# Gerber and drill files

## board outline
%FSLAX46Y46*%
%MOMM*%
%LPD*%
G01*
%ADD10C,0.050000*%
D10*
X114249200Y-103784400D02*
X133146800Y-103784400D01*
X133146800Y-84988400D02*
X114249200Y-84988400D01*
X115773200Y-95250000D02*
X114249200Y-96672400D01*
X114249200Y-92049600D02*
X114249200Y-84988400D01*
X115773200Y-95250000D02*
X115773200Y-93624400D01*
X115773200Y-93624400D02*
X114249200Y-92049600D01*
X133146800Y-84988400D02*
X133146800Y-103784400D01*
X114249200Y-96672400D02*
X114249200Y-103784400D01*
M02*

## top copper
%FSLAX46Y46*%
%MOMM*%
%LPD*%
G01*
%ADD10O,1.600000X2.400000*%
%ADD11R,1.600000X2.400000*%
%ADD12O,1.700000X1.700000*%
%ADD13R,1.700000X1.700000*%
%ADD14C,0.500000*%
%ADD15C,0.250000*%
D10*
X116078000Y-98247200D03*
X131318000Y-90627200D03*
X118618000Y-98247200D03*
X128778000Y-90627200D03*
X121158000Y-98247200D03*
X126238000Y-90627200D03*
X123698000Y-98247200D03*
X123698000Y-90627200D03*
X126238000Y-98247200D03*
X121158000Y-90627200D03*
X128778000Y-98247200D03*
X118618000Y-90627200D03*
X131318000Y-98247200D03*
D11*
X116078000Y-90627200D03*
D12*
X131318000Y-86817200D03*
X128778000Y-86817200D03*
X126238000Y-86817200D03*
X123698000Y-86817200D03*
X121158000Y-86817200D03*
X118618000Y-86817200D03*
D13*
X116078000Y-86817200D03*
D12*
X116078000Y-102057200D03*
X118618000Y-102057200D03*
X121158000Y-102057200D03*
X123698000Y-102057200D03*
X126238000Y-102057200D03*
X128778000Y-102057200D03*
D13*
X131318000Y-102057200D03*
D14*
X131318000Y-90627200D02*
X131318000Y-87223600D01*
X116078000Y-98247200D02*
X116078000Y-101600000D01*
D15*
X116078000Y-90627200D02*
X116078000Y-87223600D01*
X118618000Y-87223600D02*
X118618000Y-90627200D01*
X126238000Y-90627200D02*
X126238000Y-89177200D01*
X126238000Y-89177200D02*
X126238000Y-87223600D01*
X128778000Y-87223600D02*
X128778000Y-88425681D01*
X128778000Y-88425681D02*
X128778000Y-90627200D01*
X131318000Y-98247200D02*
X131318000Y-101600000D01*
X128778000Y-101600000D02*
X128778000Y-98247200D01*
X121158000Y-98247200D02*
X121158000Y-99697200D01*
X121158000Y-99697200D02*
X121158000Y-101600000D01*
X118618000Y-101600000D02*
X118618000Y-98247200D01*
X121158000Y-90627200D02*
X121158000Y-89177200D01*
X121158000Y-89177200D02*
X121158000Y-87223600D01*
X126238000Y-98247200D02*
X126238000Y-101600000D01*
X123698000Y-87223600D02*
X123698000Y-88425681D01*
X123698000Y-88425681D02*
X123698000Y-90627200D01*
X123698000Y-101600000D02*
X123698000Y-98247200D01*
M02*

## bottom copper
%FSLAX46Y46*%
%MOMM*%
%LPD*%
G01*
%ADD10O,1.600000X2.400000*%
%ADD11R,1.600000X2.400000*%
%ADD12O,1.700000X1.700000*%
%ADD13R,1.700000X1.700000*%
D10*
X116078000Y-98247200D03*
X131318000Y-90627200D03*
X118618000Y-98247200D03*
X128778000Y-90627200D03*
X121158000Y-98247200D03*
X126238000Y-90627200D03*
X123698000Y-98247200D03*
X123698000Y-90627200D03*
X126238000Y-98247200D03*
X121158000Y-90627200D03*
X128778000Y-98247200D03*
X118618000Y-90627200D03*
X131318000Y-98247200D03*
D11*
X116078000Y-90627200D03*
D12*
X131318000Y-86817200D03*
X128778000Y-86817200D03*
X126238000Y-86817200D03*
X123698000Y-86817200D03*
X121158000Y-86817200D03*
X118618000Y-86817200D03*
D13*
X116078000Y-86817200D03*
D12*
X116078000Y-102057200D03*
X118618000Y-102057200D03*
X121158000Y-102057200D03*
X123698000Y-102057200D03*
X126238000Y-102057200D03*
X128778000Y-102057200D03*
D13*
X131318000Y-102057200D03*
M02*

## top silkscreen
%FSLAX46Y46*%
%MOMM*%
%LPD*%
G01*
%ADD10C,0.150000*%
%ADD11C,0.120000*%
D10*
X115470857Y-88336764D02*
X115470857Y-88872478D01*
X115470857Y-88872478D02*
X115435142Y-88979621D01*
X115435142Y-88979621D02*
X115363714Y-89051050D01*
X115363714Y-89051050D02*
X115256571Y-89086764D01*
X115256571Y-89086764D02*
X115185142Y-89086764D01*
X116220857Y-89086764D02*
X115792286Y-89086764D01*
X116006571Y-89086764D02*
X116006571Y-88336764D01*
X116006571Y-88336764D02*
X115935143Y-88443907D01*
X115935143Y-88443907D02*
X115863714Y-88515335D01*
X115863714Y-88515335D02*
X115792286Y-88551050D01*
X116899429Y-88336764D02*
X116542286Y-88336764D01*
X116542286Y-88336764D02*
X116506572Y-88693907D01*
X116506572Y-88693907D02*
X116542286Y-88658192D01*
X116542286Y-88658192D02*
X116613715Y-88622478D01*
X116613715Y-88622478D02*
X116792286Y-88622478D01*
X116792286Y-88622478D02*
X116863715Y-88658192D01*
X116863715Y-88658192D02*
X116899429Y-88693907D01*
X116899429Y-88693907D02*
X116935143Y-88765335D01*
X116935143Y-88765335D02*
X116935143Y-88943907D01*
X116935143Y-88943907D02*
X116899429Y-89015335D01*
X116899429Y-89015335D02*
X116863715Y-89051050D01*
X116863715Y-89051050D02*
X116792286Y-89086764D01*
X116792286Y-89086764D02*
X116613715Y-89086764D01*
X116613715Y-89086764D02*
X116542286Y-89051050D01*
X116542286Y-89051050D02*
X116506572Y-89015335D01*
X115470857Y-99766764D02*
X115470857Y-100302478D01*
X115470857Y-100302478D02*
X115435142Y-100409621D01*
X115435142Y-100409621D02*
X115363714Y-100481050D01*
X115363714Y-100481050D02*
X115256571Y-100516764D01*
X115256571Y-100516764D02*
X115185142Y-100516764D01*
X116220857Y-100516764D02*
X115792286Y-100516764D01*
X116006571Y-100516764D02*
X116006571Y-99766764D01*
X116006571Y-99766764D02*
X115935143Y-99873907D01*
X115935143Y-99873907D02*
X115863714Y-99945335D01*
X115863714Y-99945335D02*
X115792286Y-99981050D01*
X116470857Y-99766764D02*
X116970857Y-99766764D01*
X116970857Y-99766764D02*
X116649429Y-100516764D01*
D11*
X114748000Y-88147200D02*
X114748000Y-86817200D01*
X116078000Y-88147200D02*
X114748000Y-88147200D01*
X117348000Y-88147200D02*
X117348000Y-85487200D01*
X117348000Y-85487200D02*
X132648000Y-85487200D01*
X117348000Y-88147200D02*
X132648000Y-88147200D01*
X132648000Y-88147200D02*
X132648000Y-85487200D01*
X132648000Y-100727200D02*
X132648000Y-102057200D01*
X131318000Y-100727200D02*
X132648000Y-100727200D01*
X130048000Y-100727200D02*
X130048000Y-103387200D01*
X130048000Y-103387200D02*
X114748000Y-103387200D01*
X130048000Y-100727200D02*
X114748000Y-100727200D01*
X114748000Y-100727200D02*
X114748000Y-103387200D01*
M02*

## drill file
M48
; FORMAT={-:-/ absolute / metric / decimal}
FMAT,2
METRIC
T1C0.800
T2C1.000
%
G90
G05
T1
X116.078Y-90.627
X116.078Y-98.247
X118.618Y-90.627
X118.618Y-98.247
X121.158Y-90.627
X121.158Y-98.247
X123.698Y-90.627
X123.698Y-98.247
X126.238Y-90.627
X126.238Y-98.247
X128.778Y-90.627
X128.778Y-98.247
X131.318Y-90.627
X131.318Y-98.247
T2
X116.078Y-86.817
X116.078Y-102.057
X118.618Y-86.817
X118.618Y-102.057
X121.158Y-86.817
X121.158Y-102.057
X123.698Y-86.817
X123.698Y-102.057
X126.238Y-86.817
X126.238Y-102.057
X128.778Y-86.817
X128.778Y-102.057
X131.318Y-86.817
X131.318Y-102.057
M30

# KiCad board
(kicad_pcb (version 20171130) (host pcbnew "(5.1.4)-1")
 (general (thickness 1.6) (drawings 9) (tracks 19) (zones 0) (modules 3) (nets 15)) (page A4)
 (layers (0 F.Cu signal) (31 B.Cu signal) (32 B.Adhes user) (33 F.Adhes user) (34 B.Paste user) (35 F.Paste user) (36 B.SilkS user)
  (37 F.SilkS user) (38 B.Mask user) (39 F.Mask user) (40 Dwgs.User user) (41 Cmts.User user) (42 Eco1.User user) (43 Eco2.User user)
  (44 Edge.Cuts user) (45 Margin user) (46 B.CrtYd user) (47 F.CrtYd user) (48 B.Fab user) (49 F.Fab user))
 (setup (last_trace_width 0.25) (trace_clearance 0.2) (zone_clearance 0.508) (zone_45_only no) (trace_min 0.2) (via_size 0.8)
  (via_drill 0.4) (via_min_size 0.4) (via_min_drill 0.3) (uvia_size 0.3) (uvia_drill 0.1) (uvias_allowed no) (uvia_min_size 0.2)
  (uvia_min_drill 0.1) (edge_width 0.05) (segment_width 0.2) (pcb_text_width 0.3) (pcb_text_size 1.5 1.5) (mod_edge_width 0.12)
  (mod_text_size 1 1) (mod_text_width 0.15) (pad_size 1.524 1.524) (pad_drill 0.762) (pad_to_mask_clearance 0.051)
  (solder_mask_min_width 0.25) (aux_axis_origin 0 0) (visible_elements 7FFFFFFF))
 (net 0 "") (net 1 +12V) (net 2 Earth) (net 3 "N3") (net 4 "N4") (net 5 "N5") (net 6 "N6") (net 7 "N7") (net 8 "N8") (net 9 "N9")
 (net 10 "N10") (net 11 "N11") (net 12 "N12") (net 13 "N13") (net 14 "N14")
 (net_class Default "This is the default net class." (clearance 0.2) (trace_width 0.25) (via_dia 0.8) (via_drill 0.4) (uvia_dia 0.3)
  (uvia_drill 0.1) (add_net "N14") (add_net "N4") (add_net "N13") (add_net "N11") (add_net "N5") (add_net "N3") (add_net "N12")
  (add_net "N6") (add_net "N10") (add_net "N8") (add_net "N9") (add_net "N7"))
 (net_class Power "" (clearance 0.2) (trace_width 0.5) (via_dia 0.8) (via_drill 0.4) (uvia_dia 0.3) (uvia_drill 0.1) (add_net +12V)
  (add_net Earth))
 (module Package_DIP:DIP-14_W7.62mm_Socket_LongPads (layer B.Cu) (at 116.078 90.6272 270)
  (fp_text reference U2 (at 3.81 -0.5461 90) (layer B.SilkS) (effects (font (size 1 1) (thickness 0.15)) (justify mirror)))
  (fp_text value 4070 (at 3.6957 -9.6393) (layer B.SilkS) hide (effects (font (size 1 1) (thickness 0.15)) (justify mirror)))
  (pad 14 thru_hole oval (at 7.62 0 270) (size 2.4 1.6) (drill 0.8) (layers *.Cu *.Mask) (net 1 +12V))
  (pad 7 thru_hole oval (at 0 -15.24 270) (size 2.4 1.6) (drill 0.8) (layers *.Cu *.Mask) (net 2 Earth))
  (pad 13 thru_hole oval (at 7.62 -2.54 270) (size 2.4 1.6) (drill 0.8) (layers *.Cu *.Mask) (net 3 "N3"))
  (pad 6 thru_hole oval (at 0 -12.7 270) (size 2.4 1.6) (drill 0.8) (layers *.Cu *.Mask) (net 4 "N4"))
  (pad 12 thru_hole oval (at 7.62 -5.08 270) (size 2.4 1.6) (drill 0.8) (layers *.Cu *.Mask) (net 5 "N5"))
  (pad 5 thru_hole oval (at 0 -10.16 270) (size 2.4 1.6) (drill 0.8) (layers *.Cu *.Mask) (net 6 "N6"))
  (pad 11 thru_hole oval (at 7.62 -7.62 270) (size 2.4 1.6) (drill 0.8) (layers *.Cu *.Mask) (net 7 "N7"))
  (pad 4 thru_hole oval (at 0 -7.62 270) (size 2.4 1.6) (drill 0.8) (layers *.Cu *.Mask) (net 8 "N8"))
  (pad 10 thru_hole oval (at 7.62 -10.16 270) (size 2.4 1.6) (drill 0.8) (layers *.Cu *.Mask) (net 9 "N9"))
  (pad 3 thru_hole oval (at 0 -5.08 270) (size 2.4 1.6) (drill 0.8) (layers *.Cu *.Mask) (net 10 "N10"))
  (pad 9 thru_hole oval (at 7.62 -12.7 270) (size 2.4 1.6) (drill 0.8) (layers *.Cu *.Mask) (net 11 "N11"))
  (pad 2 thru_hole oval (at 0 -2.54 270) (size 2.4 1.6) (drill 0.8) (layers *.Cu *.Mask) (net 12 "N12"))
  (pad 8 thru_hole oval (at 7.62 -15.24 270) (size 2.4 1.6) (drill 0.8) (layers *.Cu *.Mask) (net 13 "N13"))
  (pad 1 thru_hole rect (at 0 0 270) (size 2.4 1.6) (drill 0.8) (layers *.Cu *.Mask) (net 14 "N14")))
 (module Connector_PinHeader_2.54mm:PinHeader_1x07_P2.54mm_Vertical (layer F.Cu) (at 116.078 86.8172 90)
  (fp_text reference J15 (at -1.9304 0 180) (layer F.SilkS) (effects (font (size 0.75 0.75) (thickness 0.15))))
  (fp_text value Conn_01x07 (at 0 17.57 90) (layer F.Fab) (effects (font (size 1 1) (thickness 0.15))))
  (fp_line (start -1.33 -1.33) (end 0 -1.33) (layer F.SilkS) (width 0.12))
  (fp_line (start -1.33 0) (end -1.33 -1.33) (layer F.SilkS) (width 0.12))
  (fp_line (start -1.33 1.27) (end 1.33 1.27) (layer F.SilkS) (width 0.12))
  (fp_line (start 1.33 1.27) (end 1.33 16.57) (layer F.SilkS) (width 0.12))
  (fp_line (start -1.33 1.27) (end -1.33 16.57) (layer F.SilkS) (width 0.12))
  (fp_line (start -1.33 16.57) (end 1.33 16.57) (layer F.SilkS) (width 0.12))
  (pad 7 thru_hole oval (at 0 15.24 90) (size 1.7 1.7) (drill 1) (layers *.Cu *.Mask) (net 2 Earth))
  (pad 6 thru_hole oval (at 0 12.7 90) (size 1.7 1.7) (drill 1) (layers *.Cu *.Mask) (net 4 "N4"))
  (pad 5 thru_hole oval (at 0 10.16 90) (size 1.7 1.7) (drill 1) (layers *.Cu *.Mask) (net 6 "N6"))
  (pad 4 thru_hole oval (at 0 7.62 90) (size 1.7 1.7) (drill 1) (layers *.Cu *.Mask) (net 8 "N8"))
  (pad 3 thru_hole oval (at 0 5.08 90) (size 1.7 1.7) (drill 1) (layers *.Cu *.Mask) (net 10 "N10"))
  (pad 2 thru_hole oval (at 0 2.54 90) (size 1.7 1.7) (drill 1) (layers *.Cu *.Mask) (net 12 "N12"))
  (pad 1 thru_hole rect (at 0 0 90) (size 1.7 1.7) (drill 1) (layers *.Cu *.Mask) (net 14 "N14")))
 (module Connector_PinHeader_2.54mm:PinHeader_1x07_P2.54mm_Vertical (layer F.Cu) (at 131.318 102.0572 270)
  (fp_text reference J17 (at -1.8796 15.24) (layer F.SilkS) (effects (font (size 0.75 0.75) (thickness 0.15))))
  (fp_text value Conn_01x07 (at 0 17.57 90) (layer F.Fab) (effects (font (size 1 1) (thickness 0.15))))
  (fp_line (start -1.33 -1.33) (end 0 -1.33) (layer F.SilkS) (width 0.12))
  (fp_line (start -1.33 0) (end -1.33 -1.33) (layer F.SilkS) (width 0.12))
  (fp_line (start -1.33 1.27) (end 1.33 1.27) (layer F.SilkS) (width 0.12))
  (fp_line (start 1.33 1.27) (end 1.33 16.57) (layer F.SilkS) (width 0.12))
  (fp_line (start -1.33 1.27) (end -1.33 16.57) (layer F.SilkS) (width 0.12))
  (fp_line (start -1.33 16.57) (end 1.33 16.57) (layer F.SilkS) (width 0.12))
  (pad 7 thru_hole oval (at 0 15.24 270) (size 1.7 1.7) (drill 1) (layers *.Cu *.Mask) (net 1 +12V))
  (pad 6 thru_hole oval (at 0 12.7 270) (size 1.7 1.7) (drill 1) (layers *.Cu *.Mask) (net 3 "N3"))
  (pad 5 thru_hole oval (at 0 10.16 270) (size 1.7 1.7) (drill 1) (layers *.Cu *.Mask) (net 5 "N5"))
  (pad 4 thru_hole oval (at 0 7.62 270) (size 1.7 1.7) (drill 1) (layers *.Cu *.Mask) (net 7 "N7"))
  (pad 3 thru_hole oval (at 0 5.08 270) (size 1.7 1.7) (drill 1) (layers *.Cu *.Mask) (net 9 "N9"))
  (pad 2 thru_hole oval (at 0 2.54 270) (size 1.7 1.7) (drill 1) (layers *.Cu *.Mask) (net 11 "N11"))
  (pad 1 thru_hole rect (at 0 0 270) (size 1.7 1.7) (drill 1) (layers *.Cu *.Mask) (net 13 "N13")))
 (gr_line (start 114.2492 103.7844) (end 133.1468 103.7844) (layer Edge.Cuts) (width 0.05))
 (gr_line (start 133.1468 84.9884) (end 114.2492 84.9884) (layer Edge.Cuts) (width 0.05))
 (gr_line (start 115.7732 95.25) (end 114.2492 96.6724) (layer Edge.Cuts) (width 0.05))
 (gr_line (start 114.2492 92.0496) (end 114.2492 84.9884) (layer Edge.Cuts) (width 0.05))
 (gr_line (start 115.7732 95.25) (end 115.7732 93.6244) (layer Edge.Cuts) (width 0.05))
 (gr_line (start 115.7732 93.6244) (end 114.2492 92.0496) (layer Edge.Cuts) (width 0.05))
 (gr_line (start 133.1468 84.9884) (end 133.1468 103.7844) (layer Edge.Cuts) (width 0.05))
 (gr_line (start 114.2492 96.6724) (end 114.2492 103.7844) (layer Edge.Cuts) (width 0.05))
 (segment (start 131.318 90.6272) (end 131.318 87.2236) (width 0.5) (layer F.Cu) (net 2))
 (segment (start 116.078 98.2472) (end 116.078 101.6) (width 0.5) (layer F.Cu) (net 1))
 (segment (start 116.078 90.6272) (end 116.078 87.2236) (width 0.25) (layer F.Cu) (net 14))
 (segment (start 118.618 87.2236) (end 118.618 90.6272) (width 0.25) (layer F.Cu) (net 12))
 (segment (start 126.238 90.6272) (end 126.238 89.1772) (width 0.25) (layer F.Cu) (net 6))
 (segment (start 126.238 89.1772) (end 126.238 87.2236) (width 0.25) (layer F.Cu) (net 6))
 (segment (start 128.778 87.2236) (end 128.778 88.425681) (width 0.25) (layer F.Cu) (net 4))
 (segment (start 128.778 88.425681) (end 128.778 90.6272) (width 0.25) (layer F.Cu) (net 4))
 (segment (start 131.318 98.2472) (end 131.318 101.6) (width 0.25) (layer F.Cu) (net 13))
 (segment (start 128.778 101.6) (end 128.778 98.2472) (width 0.25) (layer F.Cu) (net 11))
 (segment (start 121.158 98.2472) (end 121.158 99.6972) (width 0.25) (layer F.Cu) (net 5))
 (segment (start 121.158 99.6972) (end 121.158 101.6) (width 0.25) (layer F.Cu) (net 5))
 (segment (start 118.618 101.6) (end 118.618 98.2472) (width 0.25) (layer F.Cu) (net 3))
 (segment (start 121.158 90.6272) (end 121.158 89.1772) (width 0.25) (layer F.Cu) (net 10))
 (segment (start 121.158 89.1772) (end 121.158 87.2236) (width 0.25) (layer F.Cu) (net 10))
 (segment (start 126.238 98.2472) (end 126.238 101.6) (width 0.25) (layer F.Cu) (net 9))
 (segment (start 123.698 87.2236) (end 123.698 88.425681) (width 0.25) (layer F.Cu) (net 8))
 (segment (start 123.698 88.425681) (end 123.698 90.6272) (width 0.25) (layer F.Cu) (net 8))
 (segment (start 123.698 101.6) (end 123.698 98.2472) (width 0.25) (layer F.Cu) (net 7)))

